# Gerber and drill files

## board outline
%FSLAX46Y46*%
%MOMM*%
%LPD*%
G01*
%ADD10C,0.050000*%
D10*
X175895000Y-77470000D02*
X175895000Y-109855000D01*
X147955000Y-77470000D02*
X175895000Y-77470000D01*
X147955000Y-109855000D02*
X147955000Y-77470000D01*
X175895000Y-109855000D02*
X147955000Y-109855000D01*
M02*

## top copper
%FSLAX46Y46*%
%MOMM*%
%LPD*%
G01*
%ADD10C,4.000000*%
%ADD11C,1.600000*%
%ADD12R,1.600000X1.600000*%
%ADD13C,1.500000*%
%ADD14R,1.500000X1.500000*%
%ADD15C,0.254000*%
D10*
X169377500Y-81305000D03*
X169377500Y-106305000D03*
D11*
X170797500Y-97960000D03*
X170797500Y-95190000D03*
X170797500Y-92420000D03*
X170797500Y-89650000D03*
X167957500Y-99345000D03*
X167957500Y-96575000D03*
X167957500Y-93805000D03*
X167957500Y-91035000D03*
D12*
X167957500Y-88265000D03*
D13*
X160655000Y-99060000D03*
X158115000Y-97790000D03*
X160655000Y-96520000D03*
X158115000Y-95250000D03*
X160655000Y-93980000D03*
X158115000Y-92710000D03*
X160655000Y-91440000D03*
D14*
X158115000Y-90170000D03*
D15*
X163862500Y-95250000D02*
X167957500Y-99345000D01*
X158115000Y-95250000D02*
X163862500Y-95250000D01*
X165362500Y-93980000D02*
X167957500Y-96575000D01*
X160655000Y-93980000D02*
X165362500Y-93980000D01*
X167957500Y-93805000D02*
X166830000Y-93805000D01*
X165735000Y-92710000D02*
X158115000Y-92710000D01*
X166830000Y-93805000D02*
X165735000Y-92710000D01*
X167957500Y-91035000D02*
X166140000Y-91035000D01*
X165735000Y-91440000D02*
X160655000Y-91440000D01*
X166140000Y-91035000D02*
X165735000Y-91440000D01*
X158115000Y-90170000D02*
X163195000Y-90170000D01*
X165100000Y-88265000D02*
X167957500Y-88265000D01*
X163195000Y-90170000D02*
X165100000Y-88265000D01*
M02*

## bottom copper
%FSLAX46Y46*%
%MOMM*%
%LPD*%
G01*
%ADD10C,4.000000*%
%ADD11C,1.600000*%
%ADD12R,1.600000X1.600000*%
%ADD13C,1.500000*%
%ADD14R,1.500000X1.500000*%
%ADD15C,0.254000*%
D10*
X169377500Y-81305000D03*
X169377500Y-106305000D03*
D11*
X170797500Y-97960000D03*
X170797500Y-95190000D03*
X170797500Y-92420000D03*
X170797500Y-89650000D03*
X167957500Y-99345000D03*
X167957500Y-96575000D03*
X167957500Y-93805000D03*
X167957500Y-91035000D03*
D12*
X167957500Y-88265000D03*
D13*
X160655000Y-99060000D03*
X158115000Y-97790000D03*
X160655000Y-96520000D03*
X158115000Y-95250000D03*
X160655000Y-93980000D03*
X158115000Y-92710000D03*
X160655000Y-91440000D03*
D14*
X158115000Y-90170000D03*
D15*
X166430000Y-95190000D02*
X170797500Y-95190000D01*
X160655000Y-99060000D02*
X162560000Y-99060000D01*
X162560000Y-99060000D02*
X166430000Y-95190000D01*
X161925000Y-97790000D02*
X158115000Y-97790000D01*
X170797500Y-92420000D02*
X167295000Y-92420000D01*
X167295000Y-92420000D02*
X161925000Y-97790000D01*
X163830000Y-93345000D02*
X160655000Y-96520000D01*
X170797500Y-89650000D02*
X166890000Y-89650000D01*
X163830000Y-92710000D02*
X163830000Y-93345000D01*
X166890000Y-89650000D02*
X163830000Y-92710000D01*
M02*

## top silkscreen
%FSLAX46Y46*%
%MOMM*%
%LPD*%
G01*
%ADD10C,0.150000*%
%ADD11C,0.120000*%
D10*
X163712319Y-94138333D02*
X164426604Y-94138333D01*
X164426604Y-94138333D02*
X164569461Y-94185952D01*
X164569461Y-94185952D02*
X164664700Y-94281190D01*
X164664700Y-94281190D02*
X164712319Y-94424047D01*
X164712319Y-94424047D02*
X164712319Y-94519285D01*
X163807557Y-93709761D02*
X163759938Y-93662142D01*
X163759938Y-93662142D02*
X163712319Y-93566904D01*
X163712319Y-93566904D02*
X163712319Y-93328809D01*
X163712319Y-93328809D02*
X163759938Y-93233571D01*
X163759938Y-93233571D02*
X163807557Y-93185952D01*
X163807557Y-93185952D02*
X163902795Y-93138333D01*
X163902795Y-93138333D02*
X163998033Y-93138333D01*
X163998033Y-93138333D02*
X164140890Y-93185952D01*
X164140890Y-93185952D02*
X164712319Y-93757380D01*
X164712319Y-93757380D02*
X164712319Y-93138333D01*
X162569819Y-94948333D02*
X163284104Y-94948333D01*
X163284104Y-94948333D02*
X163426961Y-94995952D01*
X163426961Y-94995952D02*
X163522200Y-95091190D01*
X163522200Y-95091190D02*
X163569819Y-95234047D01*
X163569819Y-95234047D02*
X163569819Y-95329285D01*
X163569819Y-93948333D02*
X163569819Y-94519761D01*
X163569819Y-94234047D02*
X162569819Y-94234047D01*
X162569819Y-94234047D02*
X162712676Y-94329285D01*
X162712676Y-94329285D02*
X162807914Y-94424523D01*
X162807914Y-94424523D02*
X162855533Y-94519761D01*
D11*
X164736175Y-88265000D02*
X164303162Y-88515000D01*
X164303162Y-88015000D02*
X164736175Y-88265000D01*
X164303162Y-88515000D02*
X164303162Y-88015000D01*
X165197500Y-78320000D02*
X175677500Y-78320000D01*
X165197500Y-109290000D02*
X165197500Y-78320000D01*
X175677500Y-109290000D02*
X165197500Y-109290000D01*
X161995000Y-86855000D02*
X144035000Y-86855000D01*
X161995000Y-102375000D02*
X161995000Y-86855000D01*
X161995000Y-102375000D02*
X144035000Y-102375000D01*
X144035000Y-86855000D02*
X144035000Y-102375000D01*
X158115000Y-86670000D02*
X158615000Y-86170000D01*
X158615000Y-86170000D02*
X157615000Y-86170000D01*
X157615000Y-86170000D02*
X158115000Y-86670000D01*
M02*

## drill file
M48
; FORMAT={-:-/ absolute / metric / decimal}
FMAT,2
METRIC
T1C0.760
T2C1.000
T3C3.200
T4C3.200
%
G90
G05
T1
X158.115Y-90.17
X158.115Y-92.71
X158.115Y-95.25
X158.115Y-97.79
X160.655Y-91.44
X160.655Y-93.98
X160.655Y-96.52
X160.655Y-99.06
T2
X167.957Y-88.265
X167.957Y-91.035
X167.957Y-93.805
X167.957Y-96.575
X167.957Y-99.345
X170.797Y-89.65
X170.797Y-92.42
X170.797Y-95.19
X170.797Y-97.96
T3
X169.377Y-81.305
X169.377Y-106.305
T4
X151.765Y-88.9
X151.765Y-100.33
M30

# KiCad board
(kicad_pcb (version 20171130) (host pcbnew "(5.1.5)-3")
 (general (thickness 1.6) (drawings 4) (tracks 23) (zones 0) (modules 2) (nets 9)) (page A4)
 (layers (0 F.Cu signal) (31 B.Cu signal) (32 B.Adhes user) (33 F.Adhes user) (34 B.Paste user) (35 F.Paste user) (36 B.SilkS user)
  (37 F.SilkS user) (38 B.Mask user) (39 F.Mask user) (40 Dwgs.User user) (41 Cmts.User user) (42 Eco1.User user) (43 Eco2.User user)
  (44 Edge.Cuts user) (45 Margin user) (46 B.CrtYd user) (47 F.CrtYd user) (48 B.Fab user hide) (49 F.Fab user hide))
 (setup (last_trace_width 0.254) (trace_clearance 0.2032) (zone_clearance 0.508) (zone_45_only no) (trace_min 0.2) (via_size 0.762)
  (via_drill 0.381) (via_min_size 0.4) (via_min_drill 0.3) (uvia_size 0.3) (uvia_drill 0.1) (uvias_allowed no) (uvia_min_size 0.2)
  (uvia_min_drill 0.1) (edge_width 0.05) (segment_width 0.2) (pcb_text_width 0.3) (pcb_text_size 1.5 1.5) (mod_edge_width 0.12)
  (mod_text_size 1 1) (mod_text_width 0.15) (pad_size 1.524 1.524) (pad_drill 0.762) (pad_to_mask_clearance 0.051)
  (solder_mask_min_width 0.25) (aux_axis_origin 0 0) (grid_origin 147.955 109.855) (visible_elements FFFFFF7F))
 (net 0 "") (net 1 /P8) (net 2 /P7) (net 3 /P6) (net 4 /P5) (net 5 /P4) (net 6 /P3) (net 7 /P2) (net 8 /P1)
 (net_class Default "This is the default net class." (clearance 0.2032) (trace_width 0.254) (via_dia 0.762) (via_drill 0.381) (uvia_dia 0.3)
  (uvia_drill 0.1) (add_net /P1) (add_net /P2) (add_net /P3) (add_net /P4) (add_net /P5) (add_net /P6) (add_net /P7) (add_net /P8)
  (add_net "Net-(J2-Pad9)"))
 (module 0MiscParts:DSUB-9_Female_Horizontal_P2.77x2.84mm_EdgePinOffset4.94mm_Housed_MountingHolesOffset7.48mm (layer F.Cu)
  (at 167.9575 88.265 90)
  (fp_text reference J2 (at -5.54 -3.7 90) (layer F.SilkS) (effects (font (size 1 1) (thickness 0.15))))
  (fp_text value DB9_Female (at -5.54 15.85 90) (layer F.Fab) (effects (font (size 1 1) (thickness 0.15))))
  (fp_line (start 0 -3.221325) (end -0.25 -3.654338) (layer F.SilkS) (width 0.12))
  (fp_line (start 0.25 -3.654338) (end 0 -3.221325) (layer F.SilkS) (width 0.12))
  (fp_line (start -0.25 -3.654338) (end 0.25 -3.654338) (layer F.SilkS) (width 0.12))
  (fp_line (start 9.945 -2.76) (end 9.945 7.72) (layer F.SilkS) (width 0.12))
  (fp_line (start -21.025 -2.76) (end 9.945 -2.76) (layer F.SilkS) (width 0.12))
  (fp_line (start -21.025 7.72) (end -21.025 -2.76) (layer F.SilkS) (width 0.12))
  (pad 0 thru_hole circle (at 6.96 1.42 90) (size 4 4) (drill 3.2) (layers *.Cu *.Mask))
  (pad 0 thru_hole circle (at -18.04 1.42 90) (size 4 4) (drill 3.2) (layers *.Cu *.Mask))
  (pad 9 thru_hole circle (at -9.695 2.84 90) (size 1.6 1.6) (drill 1) (layers *.Cu *.Mask))
  (pad 8 thru_hole circle (at -6.925 2.84 90) (size 1.6 1.6) (drill 1) (layers *.Cu *.Mask) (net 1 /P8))
  (pad 7 thru_hole circle (at -4.155 2.84 90) (size 1.6 1.6) (drill 1) (layers *.Cu *.Mask) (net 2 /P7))
  (pad 6 thru_hole circle (at -1.385 2.84 90) (size 1.6 1.6) (drill 1) (layers *.Cu *.Mask) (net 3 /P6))
  (pad 5 thru_hole circle (at -11.08 0 90) (size 1.6 1.6) (drill 1) (layers *.Cu *.Mask) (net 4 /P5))
  (pad 4 thru_hole circle (at -8.31 0 90) (size 1.6 1.6) (drill 1) (layers *.Cu *.Mask) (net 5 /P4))
  (pad 3 thru_hole circle (at -5.54 0 90) (size 1.6 1.6) (drill 1) (layers *.Cu *.Mask) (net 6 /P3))
  (pad 2 thru_hole circle (at -2.77 0 90) (size 1.6 1.6) (drill 1) (layers *.Cu *.Mask) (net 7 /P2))
  (pad 1 thru_hole rect (at 0 0 90) (size 1.6 1.6) (drill 1) (layers *.Cu *.Mask) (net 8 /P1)))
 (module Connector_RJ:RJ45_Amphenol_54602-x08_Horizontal (layer F.Cu) (at 158.115 90.17 270)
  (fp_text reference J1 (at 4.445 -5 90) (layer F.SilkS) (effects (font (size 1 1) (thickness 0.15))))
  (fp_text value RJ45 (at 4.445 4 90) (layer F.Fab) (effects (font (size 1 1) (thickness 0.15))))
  (fp_line (start -3.315 -3.88) (end -3.315 14.08) (layer F.SilkS) (width 0.12))
  (fp_line (start 12.205 -3.88) (end -3.315 -3.88) (layer F.SilkS) (width 0.12))
  (fp_line (start 12.205 -3.88) (end 12.205 14.08) (layer F.SilkS) (width 0.12))
  (fp_line (start -3.315 14.08) (end 12.205 14.08) (layer F.SilkS) (width 0.12))
  (fp_line (start -3.5 0) (end -4 -0.5) (layer F.SilkS) (width 0.12))
  (fp_line (start -4 -0.5) (end -4 0.5) (layer F.SilkS) (width 0.12))
  (fp_line (start -4 0.5) (end -3.5 0) (layer F.SilkS) (width 0.12))
  (pad 8 thru_hole circle (at 8.89 -2.54 270) (size 1.5 1.5) (drill 0.76) (layers *.Cu *.Mask) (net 1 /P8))
  (pad 7 thru_hole circle (at 7.62 0 270) (size 1.5 1.5) (drill 0.76) (layers *.Cu *.Mask) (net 2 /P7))
  (pad 6 thru_hole circle (at 6.35 -2.54 270) (size 1.5 1.5) (drill 0.76) (layers *.Cu *.Mask) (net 3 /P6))
  (pad 5 thru_hole circle (at 5.08 0 270) (size 1.5 1.5) (drill 0.76) (layers *.Cu *.Mask) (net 4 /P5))
  (pad 4 thru_hole circle (at 3.81 -2.54 270) (size 1.5 1.5) (drill 0.76) (layers *.Cu *.Mask) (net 5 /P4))
  (pad 3 thru_hole circle (at 2.54 0 270) (size 1.5 1.5) (drill 0.76) (layers *.Cu *.Mask) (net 6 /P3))
  (pad 2 thru_hole circle (at 1.27 -2.54 270) (size 1.5 1.5) (drill 0.76) (layers *.Cu *.Mask) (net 7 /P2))
  (pad 1 thru_hole rect (at 0 0 270) (size 1.5 1.5) (drill 0.76) (layers *.Cu *.Mask) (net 8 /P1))
  (pad "" np_thru_hole circle (at -1.27 6.35 270) (size 3.2 3.2) (drill 3.2) (layers *.Cu *.Mask))
  (pad "" np_thru_hole circle (at 10.16 6.35 270) (size 3.2 3.2) (drill 3.2) (layers *.Cu *.Mask)))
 (gr_line (start 175.895 77.47) (end 175.895 109.855) (layer Edge.Cuts) (width 0.05))
 (gr_line (start 147.955 77.47) (end 175.895 77.47) (layer Edge.Cuts) (width 0.05))
 (gr_line (start 147.955 109.855) (end 147.955 77.47) (layer Edge.Cuts) (width 0.05))
 (gr_line (start 175.895 109.855) (end 147.955 109.855) (layer Edge.Cuts) (width 0.05))
 (segment (start 166.43 95.19) (end 170.7975 95.19) (width 0.254) (layer B.Cu) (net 1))
 (segment (start 160.655 99.06) (end 162.56 99.06) (width 0.254) (layer B.Cu) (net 1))
 (segment (start 162.56 99.06) (end 166.43 95.19) (width 0.254) (layer B.Cu) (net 1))
 (segment (start 161.925 97.79) (end 158.115 97.79) (width 0.254) (layer B.Cu) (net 2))
 (segment (start 170.7975 92.42) (end 167.295 92.42) (width 0.254) (layer B.Cu) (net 2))
 (segment (start 167.295 92.42) (end 161.925 97.79) (width 0.254) (layer B.Cu) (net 2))
 (segment (start 163.83 93.345) (end 160.655 96.52) (width 0.254) (layer B.Cu) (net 3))
 (segment (start 170.7975 89.65) (end 166.89 89.65) (width 0.254) (layer B.Cu) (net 3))
 (segment (start 163.83 92.71) (end 163.83 93.345) (width 0.254) (layer B.Cu) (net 3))
 (segment (start 166.89 89.65) (end 163.83 92.71) (width 0.254) (layer B.Cu) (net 3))
 (segment (start 163.8625 95.25) (end 167.9575 99.345) (width 0.254) (layer F.Cu) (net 4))
 (segment (start 158.115 95.25) (end 163.8625 95.25) (width 0.254) (layer F.Cu) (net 4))
 (segment (start 165.3625 93.98) (end 167.9575 96.575) (width 0.254) (layer F.Cu) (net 5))
 (segment (start 160.655 93.98) (end 165.3625 93.98) (width 0.254) (layer F.Cu) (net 5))
 (segment (start 167.9575 93.805) (end 166.83 93.805) (width 0.254) (layer F.Cu) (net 6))
 (segment (start 165.735 92.71) (end 158.115 92.71) (width 0.254) (layer F.Cu) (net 6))
 (segment (start 166.83 93.805) (end 165.735 92.71) (width 0.254) (layer F.Cu) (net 6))
 (segment (start 167.9575 91.035) (end 166.14 91.035) (width 0.254) (layer F.Cu) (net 7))
 (segment (start 165.735 91.44) (end 160.655 91.44) (width 0.254) (layer F.Cu) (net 7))
 (segment (start 166.14 91.035) (end 165.735 91.44) (width 0.254) (layer F.Cu) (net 7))
 (segment (start 158.115 90.17) (end 163.195 90.17) (width 0.254) (layer F.Cu) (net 8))
 (segment (start 165.1 88.265) (end 167.9575 88.265) (width 0.254) (layer F.Cu) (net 8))
 (segment (start 163.195 90.17) (end 165.1 88.265) (width 0.254) (layer F.Cu) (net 8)))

